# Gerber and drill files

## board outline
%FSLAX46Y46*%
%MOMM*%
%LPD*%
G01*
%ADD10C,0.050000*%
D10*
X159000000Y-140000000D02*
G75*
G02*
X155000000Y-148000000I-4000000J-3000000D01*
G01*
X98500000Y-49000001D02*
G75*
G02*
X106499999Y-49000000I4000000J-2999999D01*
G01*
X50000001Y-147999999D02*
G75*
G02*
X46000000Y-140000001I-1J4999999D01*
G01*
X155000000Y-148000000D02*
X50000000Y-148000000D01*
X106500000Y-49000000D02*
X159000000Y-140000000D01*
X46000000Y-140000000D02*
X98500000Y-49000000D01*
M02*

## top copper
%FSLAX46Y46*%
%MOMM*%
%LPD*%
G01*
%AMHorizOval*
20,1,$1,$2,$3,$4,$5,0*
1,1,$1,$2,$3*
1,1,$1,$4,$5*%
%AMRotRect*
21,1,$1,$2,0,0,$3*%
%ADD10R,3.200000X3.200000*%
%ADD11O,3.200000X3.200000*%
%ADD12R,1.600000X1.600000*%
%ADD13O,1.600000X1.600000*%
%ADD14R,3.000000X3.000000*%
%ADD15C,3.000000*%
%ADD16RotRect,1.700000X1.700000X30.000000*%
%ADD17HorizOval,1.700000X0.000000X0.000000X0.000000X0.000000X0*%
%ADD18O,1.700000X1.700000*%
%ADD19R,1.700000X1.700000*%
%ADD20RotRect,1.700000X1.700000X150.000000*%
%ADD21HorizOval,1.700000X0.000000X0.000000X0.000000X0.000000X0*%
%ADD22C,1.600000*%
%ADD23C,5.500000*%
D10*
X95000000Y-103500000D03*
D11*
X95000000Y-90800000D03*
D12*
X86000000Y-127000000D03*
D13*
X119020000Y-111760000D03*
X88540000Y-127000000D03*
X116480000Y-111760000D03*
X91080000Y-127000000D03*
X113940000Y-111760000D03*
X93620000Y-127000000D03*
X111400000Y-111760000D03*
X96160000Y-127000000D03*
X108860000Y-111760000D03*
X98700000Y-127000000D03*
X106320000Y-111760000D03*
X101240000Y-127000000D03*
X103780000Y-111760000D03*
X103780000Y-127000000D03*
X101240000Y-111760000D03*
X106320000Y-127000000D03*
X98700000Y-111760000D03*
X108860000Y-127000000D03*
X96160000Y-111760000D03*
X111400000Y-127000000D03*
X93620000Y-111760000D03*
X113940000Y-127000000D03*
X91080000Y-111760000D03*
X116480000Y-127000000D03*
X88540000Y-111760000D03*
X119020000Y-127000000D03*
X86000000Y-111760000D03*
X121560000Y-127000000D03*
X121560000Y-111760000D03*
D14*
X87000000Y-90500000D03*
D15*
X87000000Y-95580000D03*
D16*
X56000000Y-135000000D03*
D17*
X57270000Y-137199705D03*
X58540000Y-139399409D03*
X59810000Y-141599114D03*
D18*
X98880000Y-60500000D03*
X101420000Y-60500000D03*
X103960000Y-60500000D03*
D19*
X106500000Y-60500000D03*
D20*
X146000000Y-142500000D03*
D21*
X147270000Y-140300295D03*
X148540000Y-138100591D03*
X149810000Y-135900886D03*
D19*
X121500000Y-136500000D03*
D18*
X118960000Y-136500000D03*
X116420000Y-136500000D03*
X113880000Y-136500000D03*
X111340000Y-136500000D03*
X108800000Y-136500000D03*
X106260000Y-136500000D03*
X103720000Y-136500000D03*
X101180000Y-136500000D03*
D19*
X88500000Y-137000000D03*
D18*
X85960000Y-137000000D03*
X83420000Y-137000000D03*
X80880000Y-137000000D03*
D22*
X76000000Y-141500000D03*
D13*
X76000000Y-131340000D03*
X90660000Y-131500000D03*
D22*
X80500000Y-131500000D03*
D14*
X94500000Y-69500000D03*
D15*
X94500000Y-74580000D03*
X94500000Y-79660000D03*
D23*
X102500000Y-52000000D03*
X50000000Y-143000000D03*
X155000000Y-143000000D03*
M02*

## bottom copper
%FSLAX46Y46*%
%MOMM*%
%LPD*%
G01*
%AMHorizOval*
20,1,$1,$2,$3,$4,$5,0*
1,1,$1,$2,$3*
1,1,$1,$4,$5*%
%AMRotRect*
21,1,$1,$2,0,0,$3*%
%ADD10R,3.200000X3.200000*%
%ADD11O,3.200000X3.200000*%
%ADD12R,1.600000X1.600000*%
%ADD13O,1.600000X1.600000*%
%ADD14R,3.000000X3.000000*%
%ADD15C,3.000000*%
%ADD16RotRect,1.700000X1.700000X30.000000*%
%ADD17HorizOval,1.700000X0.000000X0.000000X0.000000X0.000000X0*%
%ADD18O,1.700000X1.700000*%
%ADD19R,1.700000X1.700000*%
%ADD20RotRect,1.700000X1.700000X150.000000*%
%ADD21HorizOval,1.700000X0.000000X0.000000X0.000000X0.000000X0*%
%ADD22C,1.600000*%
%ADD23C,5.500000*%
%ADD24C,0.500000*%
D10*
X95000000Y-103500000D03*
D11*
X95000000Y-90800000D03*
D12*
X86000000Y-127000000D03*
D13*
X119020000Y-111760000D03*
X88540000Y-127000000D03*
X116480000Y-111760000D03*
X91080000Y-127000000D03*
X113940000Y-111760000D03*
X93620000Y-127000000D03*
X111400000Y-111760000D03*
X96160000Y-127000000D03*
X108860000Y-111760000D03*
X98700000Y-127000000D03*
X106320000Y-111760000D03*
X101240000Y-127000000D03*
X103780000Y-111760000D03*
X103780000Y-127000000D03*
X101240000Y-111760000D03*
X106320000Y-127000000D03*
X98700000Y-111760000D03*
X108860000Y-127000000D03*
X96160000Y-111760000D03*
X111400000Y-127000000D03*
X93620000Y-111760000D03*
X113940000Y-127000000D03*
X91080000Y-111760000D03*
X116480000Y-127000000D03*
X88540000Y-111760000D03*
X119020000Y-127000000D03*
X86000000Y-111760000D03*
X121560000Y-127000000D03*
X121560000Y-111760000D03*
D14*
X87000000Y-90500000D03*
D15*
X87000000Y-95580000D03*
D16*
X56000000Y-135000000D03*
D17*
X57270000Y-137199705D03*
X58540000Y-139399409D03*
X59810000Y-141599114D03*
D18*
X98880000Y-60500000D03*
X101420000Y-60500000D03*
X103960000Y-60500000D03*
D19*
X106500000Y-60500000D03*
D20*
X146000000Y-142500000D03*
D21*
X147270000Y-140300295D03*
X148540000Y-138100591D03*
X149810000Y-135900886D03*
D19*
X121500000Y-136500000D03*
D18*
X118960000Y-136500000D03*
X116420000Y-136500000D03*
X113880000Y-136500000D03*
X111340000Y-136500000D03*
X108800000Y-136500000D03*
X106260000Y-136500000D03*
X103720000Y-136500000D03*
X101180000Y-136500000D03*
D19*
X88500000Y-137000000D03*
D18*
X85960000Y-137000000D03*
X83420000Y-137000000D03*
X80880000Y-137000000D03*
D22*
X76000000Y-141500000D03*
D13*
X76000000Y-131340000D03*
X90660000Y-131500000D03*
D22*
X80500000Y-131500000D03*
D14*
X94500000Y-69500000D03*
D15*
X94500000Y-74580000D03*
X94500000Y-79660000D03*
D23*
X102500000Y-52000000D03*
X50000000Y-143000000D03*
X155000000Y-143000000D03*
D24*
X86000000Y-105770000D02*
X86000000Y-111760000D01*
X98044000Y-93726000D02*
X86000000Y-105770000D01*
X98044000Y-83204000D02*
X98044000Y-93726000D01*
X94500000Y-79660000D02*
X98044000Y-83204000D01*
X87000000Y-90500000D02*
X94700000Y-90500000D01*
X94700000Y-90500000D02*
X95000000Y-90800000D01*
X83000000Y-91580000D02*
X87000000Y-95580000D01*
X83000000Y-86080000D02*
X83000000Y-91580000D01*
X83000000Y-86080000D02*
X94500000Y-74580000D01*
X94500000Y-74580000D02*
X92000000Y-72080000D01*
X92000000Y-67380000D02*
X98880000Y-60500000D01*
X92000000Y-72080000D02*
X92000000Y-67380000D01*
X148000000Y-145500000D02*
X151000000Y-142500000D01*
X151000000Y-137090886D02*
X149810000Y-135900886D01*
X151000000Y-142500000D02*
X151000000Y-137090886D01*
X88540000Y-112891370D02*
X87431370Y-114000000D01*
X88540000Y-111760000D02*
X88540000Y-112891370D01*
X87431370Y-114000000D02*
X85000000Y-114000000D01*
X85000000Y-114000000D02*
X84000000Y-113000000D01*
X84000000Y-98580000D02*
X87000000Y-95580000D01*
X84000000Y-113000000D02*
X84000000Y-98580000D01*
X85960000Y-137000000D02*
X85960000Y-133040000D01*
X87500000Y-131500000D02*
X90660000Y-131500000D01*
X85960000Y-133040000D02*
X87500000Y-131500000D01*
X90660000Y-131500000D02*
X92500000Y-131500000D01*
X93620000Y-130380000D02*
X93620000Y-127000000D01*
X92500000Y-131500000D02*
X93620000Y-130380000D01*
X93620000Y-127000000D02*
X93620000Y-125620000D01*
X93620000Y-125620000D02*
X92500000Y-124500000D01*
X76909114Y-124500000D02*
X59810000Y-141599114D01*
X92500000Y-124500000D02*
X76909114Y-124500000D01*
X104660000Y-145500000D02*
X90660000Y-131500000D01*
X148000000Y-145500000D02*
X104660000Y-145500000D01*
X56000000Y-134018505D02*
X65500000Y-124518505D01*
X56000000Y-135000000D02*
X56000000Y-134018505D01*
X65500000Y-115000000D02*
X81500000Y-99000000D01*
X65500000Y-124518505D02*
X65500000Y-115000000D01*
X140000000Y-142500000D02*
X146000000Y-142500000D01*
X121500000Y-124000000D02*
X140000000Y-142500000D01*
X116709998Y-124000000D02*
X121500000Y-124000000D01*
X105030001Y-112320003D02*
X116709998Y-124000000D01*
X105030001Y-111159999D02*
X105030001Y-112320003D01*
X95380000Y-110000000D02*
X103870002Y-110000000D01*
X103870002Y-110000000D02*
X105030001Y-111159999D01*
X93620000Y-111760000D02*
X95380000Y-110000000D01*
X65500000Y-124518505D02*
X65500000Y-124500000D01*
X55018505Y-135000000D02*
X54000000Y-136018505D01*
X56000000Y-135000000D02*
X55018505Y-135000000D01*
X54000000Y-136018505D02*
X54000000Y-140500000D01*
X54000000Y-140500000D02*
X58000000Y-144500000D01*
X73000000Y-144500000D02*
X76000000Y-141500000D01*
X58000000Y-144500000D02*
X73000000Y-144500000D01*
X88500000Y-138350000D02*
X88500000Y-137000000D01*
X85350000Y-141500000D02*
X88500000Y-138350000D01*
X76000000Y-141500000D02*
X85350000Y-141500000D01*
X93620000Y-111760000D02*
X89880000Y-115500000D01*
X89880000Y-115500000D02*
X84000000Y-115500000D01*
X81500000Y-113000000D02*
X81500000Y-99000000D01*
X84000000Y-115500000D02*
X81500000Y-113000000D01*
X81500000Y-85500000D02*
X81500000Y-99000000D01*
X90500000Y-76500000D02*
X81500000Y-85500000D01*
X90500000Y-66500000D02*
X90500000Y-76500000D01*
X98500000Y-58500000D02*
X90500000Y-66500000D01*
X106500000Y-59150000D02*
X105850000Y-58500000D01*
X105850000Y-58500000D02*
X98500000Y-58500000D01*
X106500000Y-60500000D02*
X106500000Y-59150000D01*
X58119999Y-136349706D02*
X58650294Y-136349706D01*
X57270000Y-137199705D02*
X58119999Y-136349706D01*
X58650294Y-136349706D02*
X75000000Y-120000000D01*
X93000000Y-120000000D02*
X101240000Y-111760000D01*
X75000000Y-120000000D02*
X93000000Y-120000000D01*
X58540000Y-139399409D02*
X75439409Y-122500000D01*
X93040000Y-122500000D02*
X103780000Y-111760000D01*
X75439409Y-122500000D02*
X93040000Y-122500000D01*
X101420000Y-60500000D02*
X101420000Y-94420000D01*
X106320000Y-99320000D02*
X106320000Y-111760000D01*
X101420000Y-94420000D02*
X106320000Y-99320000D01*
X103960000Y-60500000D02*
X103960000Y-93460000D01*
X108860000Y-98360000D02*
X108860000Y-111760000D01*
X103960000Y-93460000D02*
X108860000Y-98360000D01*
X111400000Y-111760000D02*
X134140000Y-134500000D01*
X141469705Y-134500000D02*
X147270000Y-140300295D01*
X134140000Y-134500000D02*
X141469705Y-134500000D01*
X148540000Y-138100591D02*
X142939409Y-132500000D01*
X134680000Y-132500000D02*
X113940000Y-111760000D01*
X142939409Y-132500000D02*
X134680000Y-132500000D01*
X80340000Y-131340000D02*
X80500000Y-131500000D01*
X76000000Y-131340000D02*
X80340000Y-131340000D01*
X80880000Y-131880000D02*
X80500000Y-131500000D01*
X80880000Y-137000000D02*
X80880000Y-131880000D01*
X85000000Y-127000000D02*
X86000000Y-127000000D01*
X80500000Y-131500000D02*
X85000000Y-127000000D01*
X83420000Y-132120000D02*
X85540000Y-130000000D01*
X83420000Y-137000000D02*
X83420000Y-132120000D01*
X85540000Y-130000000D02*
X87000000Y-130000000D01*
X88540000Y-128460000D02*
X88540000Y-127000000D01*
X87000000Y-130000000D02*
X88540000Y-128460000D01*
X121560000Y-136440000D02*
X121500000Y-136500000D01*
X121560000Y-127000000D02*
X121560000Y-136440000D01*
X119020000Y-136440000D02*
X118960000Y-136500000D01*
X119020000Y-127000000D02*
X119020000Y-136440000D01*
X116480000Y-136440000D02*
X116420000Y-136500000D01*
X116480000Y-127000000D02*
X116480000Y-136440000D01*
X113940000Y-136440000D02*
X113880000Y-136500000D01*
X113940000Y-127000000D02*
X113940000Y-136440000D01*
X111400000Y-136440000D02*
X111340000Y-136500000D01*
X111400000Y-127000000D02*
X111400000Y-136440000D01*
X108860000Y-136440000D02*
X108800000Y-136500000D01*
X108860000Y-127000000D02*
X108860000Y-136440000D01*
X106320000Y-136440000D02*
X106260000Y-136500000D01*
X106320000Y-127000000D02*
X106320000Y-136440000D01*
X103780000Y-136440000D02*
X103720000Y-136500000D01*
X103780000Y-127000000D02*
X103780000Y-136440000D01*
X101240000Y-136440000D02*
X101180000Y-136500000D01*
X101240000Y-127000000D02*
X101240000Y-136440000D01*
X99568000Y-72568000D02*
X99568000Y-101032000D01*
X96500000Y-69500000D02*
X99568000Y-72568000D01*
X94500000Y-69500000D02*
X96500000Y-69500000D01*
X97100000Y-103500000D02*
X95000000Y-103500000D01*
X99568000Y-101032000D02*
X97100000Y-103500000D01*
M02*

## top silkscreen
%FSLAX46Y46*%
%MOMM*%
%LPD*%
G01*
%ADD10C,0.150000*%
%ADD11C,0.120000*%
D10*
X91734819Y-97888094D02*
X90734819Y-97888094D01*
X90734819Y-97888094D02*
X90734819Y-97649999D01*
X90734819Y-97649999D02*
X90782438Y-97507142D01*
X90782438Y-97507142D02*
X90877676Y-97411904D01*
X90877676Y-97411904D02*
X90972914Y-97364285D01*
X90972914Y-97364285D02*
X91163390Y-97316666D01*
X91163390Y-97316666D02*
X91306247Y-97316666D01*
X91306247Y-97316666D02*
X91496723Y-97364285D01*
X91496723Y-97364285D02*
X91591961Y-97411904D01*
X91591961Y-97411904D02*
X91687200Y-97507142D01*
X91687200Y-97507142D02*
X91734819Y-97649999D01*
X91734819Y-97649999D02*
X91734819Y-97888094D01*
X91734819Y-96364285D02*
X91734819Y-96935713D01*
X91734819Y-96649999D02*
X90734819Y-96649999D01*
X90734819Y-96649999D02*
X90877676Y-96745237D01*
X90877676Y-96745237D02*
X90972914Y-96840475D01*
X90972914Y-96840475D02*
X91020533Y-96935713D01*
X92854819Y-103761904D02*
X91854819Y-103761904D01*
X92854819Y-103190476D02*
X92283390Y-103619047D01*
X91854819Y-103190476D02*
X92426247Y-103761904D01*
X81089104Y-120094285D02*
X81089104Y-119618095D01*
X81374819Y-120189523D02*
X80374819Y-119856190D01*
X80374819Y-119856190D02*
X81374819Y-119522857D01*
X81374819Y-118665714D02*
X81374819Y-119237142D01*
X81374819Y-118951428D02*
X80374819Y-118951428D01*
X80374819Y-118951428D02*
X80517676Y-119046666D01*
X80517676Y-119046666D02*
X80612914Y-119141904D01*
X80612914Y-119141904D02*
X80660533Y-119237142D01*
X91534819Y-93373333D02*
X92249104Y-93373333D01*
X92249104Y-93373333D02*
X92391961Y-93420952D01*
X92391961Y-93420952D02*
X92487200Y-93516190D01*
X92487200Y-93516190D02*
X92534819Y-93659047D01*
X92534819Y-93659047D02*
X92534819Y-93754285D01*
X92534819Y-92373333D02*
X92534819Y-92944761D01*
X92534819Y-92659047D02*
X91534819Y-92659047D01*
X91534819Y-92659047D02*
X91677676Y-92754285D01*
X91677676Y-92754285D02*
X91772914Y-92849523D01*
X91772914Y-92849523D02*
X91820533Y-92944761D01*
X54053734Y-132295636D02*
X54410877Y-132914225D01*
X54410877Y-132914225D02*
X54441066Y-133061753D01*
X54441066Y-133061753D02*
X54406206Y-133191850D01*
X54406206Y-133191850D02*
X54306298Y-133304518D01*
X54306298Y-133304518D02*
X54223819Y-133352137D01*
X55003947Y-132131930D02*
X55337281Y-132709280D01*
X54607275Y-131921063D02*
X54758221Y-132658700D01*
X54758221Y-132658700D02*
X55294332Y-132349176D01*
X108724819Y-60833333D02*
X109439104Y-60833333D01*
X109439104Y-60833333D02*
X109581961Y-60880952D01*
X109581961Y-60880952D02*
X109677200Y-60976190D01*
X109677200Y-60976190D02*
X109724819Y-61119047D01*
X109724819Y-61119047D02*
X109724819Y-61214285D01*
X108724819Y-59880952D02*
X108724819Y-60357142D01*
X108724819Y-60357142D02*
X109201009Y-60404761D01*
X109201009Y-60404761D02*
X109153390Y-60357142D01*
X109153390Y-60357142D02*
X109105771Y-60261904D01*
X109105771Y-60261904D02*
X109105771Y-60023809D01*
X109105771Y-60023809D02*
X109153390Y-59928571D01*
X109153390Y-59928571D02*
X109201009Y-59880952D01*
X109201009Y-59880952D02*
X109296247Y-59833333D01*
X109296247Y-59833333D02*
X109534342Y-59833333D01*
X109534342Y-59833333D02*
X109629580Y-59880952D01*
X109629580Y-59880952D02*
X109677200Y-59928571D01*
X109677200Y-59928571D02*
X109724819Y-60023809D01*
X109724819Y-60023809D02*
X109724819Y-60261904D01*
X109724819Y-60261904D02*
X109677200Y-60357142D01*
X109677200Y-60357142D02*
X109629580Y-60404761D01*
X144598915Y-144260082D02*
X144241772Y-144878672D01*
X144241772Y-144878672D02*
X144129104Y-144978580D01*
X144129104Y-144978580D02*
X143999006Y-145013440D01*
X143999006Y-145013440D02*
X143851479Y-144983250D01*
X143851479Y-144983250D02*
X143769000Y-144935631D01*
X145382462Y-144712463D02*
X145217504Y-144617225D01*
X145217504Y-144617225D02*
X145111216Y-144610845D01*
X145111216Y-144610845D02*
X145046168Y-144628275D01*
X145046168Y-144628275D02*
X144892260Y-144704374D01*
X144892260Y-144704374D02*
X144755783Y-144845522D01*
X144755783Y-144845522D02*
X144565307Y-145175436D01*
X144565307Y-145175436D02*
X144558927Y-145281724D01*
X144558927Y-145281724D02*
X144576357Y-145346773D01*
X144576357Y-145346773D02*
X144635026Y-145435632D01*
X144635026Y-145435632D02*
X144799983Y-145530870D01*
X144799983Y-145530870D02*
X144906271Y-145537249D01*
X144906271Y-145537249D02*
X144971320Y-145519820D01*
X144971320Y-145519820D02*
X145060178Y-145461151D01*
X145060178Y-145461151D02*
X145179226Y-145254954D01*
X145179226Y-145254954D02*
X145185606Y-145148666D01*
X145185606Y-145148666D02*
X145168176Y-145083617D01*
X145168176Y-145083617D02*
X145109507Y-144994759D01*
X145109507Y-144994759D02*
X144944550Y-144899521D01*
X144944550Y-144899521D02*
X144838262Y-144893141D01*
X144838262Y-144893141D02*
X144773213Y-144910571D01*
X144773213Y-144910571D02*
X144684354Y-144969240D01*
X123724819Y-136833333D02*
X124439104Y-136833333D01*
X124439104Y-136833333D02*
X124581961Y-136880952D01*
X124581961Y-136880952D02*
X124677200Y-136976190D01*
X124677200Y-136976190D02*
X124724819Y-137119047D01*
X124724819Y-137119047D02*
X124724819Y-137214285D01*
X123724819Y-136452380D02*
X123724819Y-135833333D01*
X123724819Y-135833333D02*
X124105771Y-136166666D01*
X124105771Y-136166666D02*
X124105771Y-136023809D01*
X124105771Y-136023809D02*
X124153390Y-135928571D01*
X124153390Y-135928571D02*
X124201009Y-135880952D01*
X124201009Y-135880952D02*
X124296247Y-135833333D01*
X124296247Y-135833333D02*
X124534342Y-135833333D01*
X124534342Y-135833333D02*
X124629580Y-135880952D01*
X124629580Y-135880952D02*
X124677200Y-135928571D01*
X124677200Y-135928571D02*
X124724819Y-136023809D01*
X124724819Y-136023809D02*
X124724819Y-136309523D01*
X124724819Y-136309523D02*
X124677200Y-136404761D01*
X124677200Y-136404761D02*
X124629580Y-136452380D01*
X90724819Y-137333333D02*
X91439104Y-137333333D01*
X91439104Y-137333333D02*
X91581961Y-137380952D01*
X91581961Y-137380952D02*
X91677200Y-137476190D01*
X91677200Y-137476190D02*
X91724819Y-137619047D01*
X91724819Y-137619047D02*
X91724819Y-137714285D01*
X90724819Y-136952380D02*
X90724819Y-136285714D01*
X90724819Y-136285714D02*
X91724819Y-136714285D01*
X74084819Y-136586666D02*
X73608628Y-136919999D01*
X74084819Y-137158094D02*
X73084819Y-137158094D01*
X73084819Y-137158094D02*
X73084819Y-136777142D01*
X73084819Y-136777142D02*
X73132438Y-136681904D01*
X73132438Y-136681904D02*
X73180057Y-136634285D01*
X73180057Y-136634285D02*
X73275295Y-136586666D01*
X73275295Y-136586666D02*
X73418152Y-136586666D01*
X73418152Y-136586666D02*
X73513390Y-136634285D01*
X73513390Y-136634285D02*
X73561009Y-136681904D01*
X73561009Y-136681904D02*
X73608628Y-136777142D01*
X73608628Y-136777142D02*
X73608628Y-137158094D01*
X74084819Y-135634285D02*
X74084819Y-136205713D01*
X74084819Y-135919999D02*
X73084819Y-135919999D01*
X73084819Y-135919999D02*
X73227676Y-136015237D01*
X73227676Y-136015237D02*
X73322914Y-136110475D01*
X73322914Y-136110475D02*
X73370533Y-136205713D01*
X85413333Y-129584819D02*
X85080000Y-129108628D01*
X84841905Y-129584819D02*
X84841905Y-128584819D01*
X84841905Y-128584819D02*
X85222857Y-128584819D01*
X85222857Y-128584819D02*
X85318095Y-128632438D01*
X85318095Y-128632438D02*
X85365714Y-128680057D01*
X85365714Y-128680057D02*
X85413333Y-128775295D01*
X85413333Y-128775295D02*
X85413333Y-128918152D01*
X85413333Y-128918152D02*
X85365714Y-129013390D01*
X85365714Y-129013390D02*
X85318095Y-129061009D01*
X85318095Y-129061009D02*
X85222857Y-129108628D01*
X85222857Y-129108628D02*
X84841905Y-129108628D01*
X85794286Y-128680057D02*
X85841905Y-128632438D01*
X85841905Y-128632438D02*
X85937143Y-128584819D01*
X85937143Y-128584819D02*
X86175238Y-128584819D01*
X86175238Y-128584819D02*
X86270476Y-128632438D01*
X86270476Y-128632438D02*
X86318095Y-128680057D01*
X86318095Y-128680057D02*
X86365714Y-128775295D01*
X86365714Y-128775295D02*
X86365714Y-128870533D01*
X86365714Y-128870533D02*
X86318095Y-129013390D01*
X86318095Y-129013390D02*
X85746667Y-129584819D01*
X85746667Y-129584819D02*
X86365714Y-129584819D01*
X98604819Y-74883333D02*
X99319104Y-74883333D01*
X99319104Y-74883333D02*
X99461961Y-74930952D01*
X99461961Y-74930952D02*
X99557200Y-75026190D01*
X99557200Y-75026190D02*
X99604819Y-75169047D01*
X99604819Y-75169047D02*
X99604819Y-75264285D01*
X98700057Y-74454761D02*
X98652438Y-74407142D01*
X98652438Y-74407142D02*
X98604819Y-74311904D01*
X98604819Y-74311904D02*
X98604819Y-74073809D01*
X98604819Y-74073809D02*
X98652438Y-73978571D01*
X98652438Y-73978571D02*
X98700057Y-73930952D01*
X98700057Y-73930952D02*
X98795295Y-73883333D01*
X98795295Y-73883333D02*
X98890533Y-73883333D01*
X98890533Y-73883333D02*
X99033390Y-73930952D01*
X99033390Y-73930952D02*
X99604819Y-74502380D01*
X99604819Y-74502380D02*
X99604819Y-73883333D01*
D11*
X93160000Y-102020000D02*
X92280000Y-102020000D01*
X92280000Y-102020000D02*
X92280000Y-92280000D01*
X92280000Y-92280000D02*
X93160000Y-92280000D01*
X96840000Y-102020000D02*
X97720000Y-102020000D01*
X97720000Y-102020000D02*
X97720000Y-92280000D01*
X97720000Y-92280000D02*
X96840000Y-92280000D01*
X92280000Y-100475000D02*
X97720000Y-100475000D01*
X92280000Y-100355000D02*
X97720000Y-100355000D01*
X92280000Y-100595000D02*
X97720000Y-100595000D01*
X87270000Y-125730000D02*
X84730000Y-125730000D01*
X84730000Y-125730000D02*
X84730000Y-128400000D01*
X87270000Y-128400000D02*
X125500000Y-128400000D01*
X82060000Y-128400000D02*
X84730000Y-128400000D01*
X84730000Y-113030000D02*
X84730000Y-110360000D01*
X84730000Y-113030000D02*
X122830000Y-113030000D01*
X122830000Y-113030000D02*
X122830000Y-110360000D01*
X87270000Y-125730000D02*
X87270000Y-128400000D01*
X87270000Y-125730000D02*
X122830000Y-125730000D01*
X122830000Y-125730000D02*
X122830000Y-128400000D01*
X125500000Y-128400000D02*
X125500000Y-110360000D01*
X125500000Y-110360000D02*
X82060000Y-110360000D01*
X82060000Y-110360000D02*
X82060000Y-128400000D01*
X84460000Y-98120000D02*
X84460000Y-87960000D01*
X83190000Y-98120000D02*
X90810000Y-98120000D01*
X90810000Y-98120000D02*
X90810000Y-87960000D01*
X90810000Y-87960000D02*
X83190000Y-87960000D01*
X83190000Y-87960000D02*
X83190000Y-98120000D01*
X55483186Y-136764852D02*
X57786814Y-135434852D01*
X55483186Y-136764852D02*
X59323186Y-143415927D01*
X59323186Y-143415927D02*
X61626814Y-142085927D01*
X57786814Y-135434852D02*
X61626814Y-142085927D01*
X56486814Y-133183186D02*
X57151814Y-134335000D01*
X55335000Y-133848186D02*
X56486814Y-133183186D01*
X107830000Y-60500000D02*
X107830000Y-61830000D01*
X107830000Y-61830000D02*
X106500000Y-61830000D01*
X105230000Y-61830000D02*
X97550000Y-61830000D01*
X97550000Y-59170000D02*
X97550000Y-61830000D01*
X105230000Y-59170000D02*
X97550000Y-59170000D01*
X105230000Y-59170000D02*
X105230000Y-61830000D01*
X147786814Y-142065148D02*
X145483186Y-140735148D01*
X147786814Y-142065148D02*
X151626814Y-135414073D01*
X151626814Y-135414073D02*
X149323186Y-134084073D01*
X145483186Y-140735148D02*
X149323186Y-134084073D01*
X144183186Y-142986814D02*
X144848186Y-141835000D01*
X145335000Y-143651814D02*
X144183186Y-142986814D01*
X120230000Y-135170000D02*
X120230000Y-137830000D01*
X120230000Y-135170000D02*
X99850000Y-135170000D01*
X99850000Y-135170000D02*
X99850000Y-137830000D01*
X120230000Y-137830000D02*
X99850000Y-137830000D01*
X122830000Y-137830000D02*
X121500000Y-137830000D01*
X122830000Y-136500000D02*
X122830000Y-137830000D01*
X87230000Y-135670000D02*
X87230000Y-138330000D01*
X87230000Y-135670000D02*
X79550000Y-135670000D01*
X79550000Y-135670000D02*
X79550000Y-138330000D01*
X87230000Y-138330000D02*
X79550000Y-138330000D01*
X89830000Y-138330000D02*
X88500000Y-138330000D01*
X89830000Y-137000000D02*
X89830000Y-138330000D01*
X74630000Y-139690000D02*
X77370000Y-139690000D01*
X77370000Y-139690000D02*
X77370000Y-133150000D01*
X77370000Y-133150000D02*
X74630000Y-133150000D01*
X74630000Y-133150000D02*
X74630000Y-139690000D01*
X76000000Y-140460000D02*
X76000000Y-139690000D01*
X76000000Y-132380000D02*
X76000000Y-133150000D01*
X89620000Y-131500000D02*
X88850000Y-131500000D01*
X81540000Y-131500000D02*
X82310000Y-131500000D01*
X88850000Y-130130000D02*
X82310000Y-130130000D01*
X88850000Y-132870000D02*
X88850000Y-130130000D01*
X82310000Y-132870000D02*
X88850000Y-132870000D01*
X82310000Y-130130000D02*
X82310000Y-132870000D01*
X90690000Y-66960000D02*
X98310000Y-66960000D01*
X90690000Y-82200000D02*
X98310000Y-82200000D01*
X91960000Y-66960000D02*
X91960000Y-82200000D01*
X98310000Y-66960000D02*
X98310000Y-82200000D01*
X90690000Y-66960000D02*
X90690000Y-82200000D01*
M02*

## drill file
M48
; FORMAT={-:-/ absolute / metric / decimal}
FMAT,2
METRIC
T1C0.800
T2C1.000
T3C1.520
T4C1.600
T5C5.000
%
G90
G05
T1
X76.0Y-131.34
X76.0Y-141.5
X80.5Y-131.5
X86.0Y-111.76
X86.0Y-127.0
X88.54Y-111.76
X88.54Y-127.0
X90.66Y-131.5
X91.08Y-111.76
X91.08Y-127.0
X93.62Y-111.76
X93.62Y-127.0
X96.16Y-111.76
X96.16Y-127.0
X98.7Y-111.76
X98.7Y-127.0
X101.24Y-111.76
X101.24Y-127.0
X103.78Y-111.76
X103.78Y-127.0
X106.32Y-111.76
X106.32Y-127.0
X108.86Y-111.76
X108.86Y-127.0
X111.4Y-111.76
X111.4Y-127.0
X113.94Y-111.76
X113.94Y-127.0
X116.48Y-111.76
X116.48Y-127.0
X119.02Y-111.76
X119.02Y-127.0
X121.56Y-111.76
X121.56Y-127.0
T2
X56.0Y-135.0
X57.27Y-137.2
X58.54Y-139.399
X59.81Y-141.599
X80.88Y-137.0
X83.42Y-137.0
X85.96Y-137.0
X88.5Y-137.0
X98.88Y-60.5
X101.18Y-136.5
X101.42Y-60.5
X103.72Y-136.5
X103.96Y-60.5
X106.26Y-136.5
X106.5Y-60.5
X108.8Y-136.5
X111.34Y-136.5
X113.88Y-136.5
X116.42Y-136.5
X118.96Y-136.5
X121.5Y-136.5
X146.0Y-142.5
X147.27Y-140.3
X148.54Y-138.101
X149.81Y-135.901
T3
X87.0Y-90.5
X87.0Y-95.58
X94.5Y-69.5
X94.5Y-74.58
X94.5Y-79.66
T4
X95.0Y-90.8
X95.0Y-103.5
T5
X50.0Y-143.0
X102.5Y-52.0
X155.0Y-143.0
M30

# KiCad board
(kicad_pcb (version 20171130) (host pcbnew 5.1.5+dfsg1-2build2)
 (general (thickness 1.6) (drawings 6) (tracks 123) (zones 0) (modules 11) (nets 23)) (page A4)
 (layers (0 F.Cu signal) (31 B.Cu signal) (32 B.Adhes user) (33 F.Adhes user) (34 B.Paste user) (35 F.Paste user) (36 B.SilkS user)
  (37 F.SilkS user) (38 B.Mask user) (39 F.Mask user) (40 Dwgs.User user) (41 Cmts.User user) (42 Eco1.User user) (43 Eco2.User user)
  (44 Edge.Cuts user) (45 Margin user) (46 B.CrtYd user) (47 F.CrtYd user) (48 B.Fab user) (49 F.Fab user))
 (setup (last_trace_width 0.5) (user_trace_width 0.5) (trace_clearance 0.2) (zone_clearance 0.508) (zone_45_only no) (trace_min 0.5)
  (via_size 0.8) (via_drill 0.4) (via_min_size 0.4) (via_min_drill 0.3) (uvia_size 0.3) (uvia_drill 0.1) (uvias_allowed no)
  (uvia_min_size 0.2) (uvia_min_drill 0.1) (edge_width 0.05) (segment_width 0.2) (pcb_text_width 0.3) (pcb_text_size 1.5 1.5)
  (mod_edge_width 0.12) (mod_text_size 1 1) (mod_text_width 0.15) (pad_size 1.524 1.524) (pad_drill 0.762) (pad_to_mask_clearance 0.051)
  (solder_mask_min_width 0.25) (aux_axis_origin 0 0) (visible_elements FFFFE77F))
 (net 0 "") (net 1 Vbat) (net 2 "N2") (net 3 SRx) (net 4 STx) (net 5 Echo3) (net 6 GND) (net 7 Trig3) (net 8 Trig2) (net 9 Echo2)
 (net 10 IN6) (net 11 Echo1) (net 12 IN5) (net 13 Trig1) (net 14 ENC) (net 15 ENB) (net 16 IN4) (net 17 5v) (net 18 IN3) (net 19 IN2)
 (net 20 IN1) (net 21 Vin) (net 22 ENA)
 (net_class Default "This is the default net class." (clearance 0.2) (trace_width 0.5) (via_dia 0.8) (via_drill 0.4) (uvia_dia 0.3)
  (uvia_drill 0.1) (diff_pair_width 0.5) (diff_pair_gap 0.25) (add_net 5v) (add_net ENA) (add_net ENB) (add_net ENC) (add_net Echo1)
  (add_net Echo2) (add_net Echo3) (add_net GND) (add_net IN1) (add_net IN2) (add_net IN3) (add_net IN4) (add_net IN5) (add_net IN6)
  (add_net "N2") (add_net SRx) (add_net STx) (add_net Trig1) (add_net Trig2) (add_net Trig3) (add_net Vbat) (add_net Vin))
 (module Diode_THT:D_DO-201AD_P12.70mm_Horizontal (layer F.Cu) (at 95 103.5 90)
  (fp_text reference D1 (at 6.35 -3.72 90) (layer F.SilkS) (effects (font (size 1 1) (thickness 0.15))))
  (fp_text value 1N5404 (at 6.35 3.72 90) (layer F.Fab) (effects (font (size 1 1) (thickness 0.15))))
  (fp_line (start 1.48 -1.84) (end 1.48 -2.72) (layer F.SilkS) (width 0.12))
  (fp_line (start 1.48 -2.72) (end 11.22 -2.72) (layer F.SilkS) (width 0.12))
  (fp_line (start 11.22 -2.72) (end 11.22 -1.84) (layer F.SilkS) (width 0.12))
  (fp_line (start 1.48 1.84) (end 1.48 2.72) (layer F.SilkS) (width 0.12))
  (fp_line (start 1.48 2.72) (end 11.22 2.72) (layer F.SilkS) (width 0.12))
  (fp_line (start 11.22 2.72) (end 11.22 1.84) (layer F.SilkS) (width 0.12))
  (fp_line (start 3.025 -2.72) (end 3.025 2.72) (layer F.SilkS) (width 0.12))
  (fp_line (start 3.145 -2.72) (end 3.145 2.72) (layer F.SilkS) (width 0.12))
  (fp_line (start 2.905 -2.72) (end 2.905 2.72) (layer F.SilkS) (width 0.12))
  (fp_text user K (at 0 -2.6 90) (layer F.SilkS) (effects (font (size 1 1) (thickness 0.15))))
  (pad 1 thru_hole rect (at 0 0 90) (size 3.2 3.2) (drill 1.6) (layers *.Cu *.Mask) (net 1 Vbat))
  (pad 2 thru_hole oval (at 12.7 0 90) (size 3.2 3.2) (drill 1.6) (layers *.Cu *.Mask) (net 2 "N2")))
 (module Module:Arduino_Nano (layer F.Cu) (at 86 127 90)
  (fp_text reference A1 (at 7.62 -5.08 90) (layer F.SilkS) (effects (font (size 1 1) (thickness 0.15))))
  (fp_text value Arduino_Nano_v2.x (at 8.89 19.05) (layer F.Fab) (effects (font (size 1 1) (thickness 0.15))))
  (fp_line (start 1.27 1.27) (end 1.27 -1.27) (layer F.SilkS) (width 0.12))
  (fp_line (start 1.27 -1.27) (end -1.4 -1.27) (layer F.SilkS) (width 0.12))
  (fp_line (start -1.4 1.27) (end -1.4 39.5) (layer F.SilkS) (width 0.12))
  (fp_line (start -1.4 -3.94) (end -1.4 -1.27) (layer F.SilkS) (width 0.12))
  (fp_line (start 13.97 -1.27) (end 16.64 -1.27) (layer F.SilkS) (width 0.12))
  (fp_line (start 13.97 -1.27) (end 13.97 36.83) (layer F.SilkS) (width 0.12))
  (fp_line (start 13.97 36.83) (end 16.64 36.83) (layer F.SilkS) (width 0.12))
  (fp_line (start 1.27 1.27) (end -1.4 1.27) (layer F.SilkS) (width 0.12))
  (fp_line (start 1.27 1.27) (end 1.27 36.83) (layer F.SilkS) (width 0.12))
  (fp_line (start 1.27 36.83) (end -1.4 36.83) (layer F.SilkS) (width 0.12))
  (fp_line (start -1.4 39.5) (end 16.64 39.5) (layer F.SilkS) (width 0.12))
  (fp_line (start 16.64 39.5) (end 16.64 -3.94) (layer F.SilkS) (width 0.12))
  (fp_line (start 16.64 -3.94) (end -1.4 -3.94) (layer F.SilkS) (width 0.12))
  (pad 1 thru_hole rect (at 0 0 90) (size 1.6 1.6) (drill 0.8) (layers *.Cu *.Mask) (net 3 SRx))
  (pad 17 thru_hole oval (at 15.24 33.02 90) (size 1.6 1.6) (drill 0.8) (layers *.Cu *.Mask))
  (pad 2 thru_hole oval (at 0 2.54 90) (size 1.6 1.6) (drill 0.8) (layers *.Cu *.Mask) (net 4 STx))
  (pad 18 thru_hole oval (at 15.24 30.48 90) (size 1.6 1.6) (drill 0.8) (layers *.Cu *.Mask))
  (pad 3 thru_hole oval (at 0 5.08 90) (size 1.6 1.6) (drill 0.8) (layers *.Cu *.Mask))
  (pad 19 thru_hole oval (at 15.24 27.94 90) (size 1.6 1.6) (drill 0.8) (layers *.Cu *.Mask) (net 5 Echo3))
  (pad 4 thru_hole oval (at 0 7.62 90) (size 1.6 1.6) (drill 0.8) (layers *.Cu *.Mask) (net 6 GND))
  (pad 20 thru_hole oval (at 15.24 25.4 90) (size 1.6 1.6) (drill 0.8) (layers *.Cu *.Mask) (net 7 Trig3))
  (pad 5 thru_hole oval (at 0 10.16 90) (size 1.6 1.6) (drill 0.8) (layers *.Cu *.Mask))
  (pad 21 thru_hole oval (at 15.24 22.86 90) (size 1.6 1.6) (drill 0.8) (layers *.Cu *.Mask) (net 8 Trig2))
  (pad 6 thru_hole oval (at 0 12.7 90) (size 1.6 1.6) (drill 0.8) (layers *.Cu *.Mask))
  (pad 22 thru_hole oval (at 15.24 20.32 90) (size 1.6 1.6) (drill 0.8) (layers *.Cu *.Mask) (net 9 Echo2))
  (pad 7 thru_hole oval (at 0 15.24 90) (size 1.6 1.6) (drill 0.8) (layers *.Cu *.Mask) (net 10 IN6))
  (pad 23 thru_hole oval (at 15.24 17.78 90) (size 1.6 1.6) (drill 0.8) (layers *.Cu *.Mask) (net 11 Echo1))
  (pad 8 thru_hole oval (at 0 17.78 90) (size 1.6 1.6) (drill 0.8) (layers *.Cu *.Mask) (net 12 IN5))
  (pad 24 thru_hole oval (at 15.24 15.24 90) (size 1.6 1.6) (drill 0.8) (layers *.Cu *.Mask) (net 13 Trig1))
  (pad 9 thru_hole oval (at 0 20.32 90) (size 1.6 1.6) (drill 0.8) (layers *.Cu *.Mask) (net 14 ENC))
  (pad 25 thru_hole oval (at 15.24 12.7 90) (size 1.6 1.6) (drill 0.8) (layers *.Cu *.Mask))
  (pad 10 thru_hole oval (at 0 22.86 90) (size 1.6 1.6) (drill 0.8) (layers *.Cu *.Mask) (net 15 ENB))
  (pad 26 thru_hole oval (at 15.24 10.16 90) (size 1.6 1.6) (drill 0.8) (layers *.Cu *.Mask))
  (pad 11 thru_hole oval (at 0 25.4 90) (size 1.6 1.6) (drill 0.8) (layers *.Cu *.Mask) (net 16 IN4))
  (pad 27 thru_hole oval (at 15.24 7.62 90) (size 1.6 1.6) (drill 0.8) (layers *.Cu *.Mask) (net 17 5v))
  (pad 12 thru_hole oval (at 0 27.94 90) (size 1.6 1.6) (drill 0.8) (layers *.Cu *.Mask) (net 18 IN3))
  (pad 28 thru_hole oval (at 15.24 5.08 90) (size 1.6 1.6) (drill 0.8) (layers *.Cu *.Mask))
  (pad 13 thru_hole oval (at 0 30.48 90) (size 1.6 1.6) (drill 0.8) (layers *.Cu *.Mask) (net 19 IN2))
  (pad 29 thru_hole oval (at 15.24 2.54 90) (size 1.6 1.6) (drill 0.8) (layers *.Cu *.Mask) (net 6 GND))
  (pad 14 thru_hole oval (at 0 33.02 90) (size 1.6 1.6) (drill 0.8) (layers *.Cu *.Mask) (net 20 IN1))
  (pad 30 thru_hole oval (at 15.24 0 90) (size 1.6 1.6) (drill 0.8) (layers *.Cu *.Mask) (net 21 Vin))
  (pad 15 thru_hole oval (at 0 35.56 90) (size 1.6 1.6) (drill 0.8) (layers *.Cu *.Mask) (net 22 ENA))
  (pad 16 thru_hole oval (at 15.24 35.56 90) (size 1.6 1.6) (drill 0.8) (layers *.Cu *.Mask)))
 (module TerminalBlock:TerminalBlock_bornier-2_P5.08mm (layer F.Cu) (at 87 90.5 270)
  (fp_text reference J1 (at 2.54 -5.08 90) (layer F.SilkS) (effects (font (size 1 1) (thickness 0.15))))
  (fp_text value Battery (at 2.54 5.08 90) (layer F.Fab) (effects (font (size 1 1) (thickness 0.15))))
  (fp_line (start 7.62 2.54) (end -2.54 2.54) (layer F.SilkS) (width 0.12))
  (fp_line (start 7.62 3.81) (end 7.62 -3.81) (layer F.SilkS) (width 0.12))
  (fp_line (start 7.62 -3.81) (end -2.54 -3.81) (layer F.SilkS) (width 0.12))
  (fp_line (start -2.54 -3.81) (end -2.54 3.81) (layer F.SilkS) (width 0.12))
  (fp_line (start -2.54 3.81) (end 7.62 3.81) (layer F.SilkS) (width 0.12))
  (pad 1 thru_hole rect (at 0 0 270) (size 3 3) (drill 1.52) (layers *.Cu *.Mask) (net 2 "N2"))
  (pad 2 thru_hole circle (at 5.08 0 270) (size 3 3) (drill 1.52) (layers *.Cu *.Mask) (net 6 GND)))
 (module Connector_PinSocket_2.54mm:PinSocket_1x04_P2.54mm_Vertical (layer F.Cu) (at 56 135 30)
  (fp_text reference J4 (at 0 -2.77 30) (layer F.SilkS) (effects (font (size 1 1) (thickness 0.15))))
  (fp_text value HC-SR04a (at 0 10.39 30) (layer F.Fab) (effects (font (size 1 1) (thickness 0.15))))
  (fp_line (start -1.33 1.27) (end 1.33 1.27) (layer F.SilkS) (width 0.12))
  (fp_line (start -1.33 1.27) (end -1.33 8.95) (layer F.SilkS) (width 0.12))
  (fp_line (start -1.33 8.95) (end 1.33 8.95) (layer F.SilkS) (width 0.12))
  (fp_line (start 1.33 1.27) (end 1.33 8.95) (layer F.SilkS) (width 0.12))
  (fp_line (start 1.33 -1.33) (end 1.33 0) (layer F.SilkS) (width 0.12))
  (fp_line (start 0 -1.33) (end 1.33 -1.33) (layer F.SilkS) (width 0.12))
  (pad 1 thru_hole rect (at 0 0 30) (size 1.7 1.7) (drill 1) (layers *.Cu *.Mask) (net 17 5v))
  (pad 2 thru_hole oval (at 0 2.54 30) (size 1.7 1.7) (drill 1) (layers *.Cu *.Mask) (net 13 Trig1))
  (pad 3 thru_hole oval (at 0 5.08 30) (size 1.7 1.7) (drill 1) (layers *.Cu *.Mask) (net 11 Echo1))
  (pad 4 thru_hole oval (at 0 7.62 30) (size 1.7 1.7) (drill 1) (layers *.Cu *.Mask) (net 6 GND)))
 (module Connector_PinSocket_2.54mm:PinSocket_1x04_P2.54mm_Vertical (layer F.Cu) (at 106.5 60.5 270)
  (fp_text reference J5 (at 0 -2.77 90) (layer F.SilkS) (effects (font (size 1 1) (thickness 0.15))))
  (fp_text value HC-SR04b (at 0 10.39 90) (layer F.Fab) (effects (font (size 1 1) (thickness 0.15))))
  (fp_line (start 0 -1.33) (end 1.33 -1.33) (layer F.SilkS) (width 0.12))
  (fp_line (start 1.33 -1.33) (end 1.33 0) (layer F.SilkS) (width 0.12))
  (fp_line (start 1.33 1.27) (end 1.33 8.95) (layer F.SilkS) (width 0.12))
  (fp_line (start -1.33 8.95) (end 1.33 8.95) (layer F.SilkS) (width 0.12))
  (fp_line (start -1.33 1.27) (end -1.33 8.95) (layer F.SilkS) (width 0.12))
  (fp_line (start -1.33 1.27) (end 1.33 1.27) (layer F.SilkS) (width 0.12))
  (pad 4 thru_hole oval (at 0 7.62 270) (size 1.7 1.7) (drill 1) (layers *.Cu *.Mask) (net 6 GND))
  (pad 3 thru_hole oval (at 0 5.08 270) (size 1.7 1.7) (drill 1) (layers *.Cu *.Mask) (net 9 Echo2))
  (pad 2 thru_hole oval (at 0 2.54 270) (size 1.7 1.7) (drill 1) (layers *.Cu *.Mask) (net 8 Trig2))
  (pad 1 thru_hole rect (at 0 0 270) (size 1.7 1.7) (drill 1) (layers *.Cu *.Mask) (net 17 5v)))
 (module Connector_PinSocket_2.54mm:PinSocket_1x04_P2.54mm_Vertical (layer F.Cu) (at 146 142.5 150)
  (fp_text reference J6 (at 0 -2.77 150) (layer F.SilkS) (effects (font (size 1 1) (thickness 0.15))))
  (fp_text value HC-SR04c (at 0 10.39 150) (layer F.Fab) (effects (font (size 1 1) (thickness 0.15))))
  (fp_line (start -1.33 1.27) (end 1.33 1.27) (layer F.SilkS) (width 0.12))
  (fp_line (start -1.33 1.27) (end -1.33 8.95) (layer F.SilkS) (width 0.12))
  (fp_line (start -1.33 8.95) (end 1.33 8.95) (layer F.SilkS) (width 0.12))
  (fp_line (start 1.33 1.27) (end 1.33 8.95) (layer F.SilkS) (width 0.12))
  (fp_line (start 1.33 -1.33) (end 1.33 0) (layer F.SilkS) (width 0.12))
  (fp_line (start 0 -1.33) (end 1.33 -1.33) (layer F.SilkS) (width 0.12))
  (pad 1 thru_hole rect (at 0 0 150) (size 1.7 1.7) (drill 1) (layers *.Cu *.Mask) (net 17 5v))
  (pad 2 thru_hole oval (at 0 2.54 150) (size 1.7 1.7) (drill 1) (layers *.Cu *.Mask) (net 7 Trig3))
  (pad 3 thru_hole oval (at 0 5.08 150) (size 1.7 1.7) (drill 1) (layers *.Cu *.Mask) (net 5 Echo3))
  (pad 4 thru_hole oval (at 0 7.62 150) (size 1.7 1.7) (drill 1) (layers *.Cu *.Mask) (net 6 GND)))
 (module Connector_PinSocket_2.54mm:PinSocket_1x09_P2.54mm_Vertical (layer F.Cu) (at 121.5 136.5 270)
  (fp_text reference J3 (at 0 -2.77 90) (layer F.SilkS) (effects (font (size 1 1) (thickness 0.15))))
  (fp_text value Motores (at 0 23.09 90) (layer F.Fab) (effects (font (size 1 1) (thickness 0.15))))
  (fp_line (start -1.33 1.27) (end 1.33 1.27) (layer F.SilkS) (width 0.12))
  (fp_line (start -1.33 1.27) (end -1.33 21.65) (layer F.SilkS) (width 0.12))
  (fp_line (start -1.33 21.65) (end 1.33 21.65) (layer F.SilkS) (width 0.12))
  (fp_line (start 1.33 1.27) (end 1.33 21.65) (layer F.SilkS) (width 0.12))
  (fp_line (start 1.33 -1.33) (end 1.33 0) (layer F.SilkS) (width 0.12))
  (fp_line (start 0 -1.33) (end 1.33 -1.33) (layer F.SilkS) (width 0.12))
  (pad 1 thru_hole rect (at 0 0 270) (size 1.7 1.7) (drill 1) (layers *.Cu *.Mask) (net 22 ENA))
  (pad 2 thru_hole oval (at 0 2.54 270) (size 1.7 1.7) (drill 1) (layers *.Cu *.Mask) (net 20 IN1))
  (pad 3 thru_hole oval (at 0 5.08 270) (size 1.7 1.7) (drill 1) (layers *.Cu *.Mask) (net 19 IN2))
  (pad 4 thru_hole oval (at 0 7.62 270) (size 1.7 1.7) (drill 1) (layers *.Cu *.Mask) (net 18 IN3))
  (pad 5 thru_hole oval (at 0 10.16 270) (size 1.7 1.7) (drill 1) (layers *.Cu *.Mask) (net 16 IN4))
  (pad 6 thru_hole oval (at 0 12.7 270) (size 1.7 1.7) (drill 1) (layers *.Cu *.Mask) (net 15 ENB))
  (pad 7 thru_hole oval (at 0 15.24 270) (size 1.7 1.7) (drill 1) (layers *.Cu *.Mask) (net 14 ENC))
  (pad 8 thru_hole oval (at 0 17.78 270) (size 1.7 1.7) (drill 1) (layers *.Cu *.Mask) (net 12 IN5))
  (pad 9 thru_hole oval (at 0 20.32 270) (size 1.7 1.7) (drill 1) (layers *.Cu *.Mask) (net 10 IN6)))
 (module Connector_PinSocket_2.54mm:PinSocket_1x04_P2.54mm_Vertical (layer F.Cu) (at 88.5 137 270)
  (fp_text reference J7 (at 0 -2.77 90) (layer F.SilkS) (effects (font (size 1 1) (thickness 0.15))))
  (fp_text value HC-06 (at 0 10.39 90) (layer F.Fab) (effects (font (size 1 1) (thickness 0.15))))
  (fp_line (start -1.33 1.27) (end 1.33 1.27) (layer F.SilkS) (width 0.12))
  (fp_line (start -1.33 1.27) (end -1.33 8.95) (layer F.SilkS) (width 0.12))
  (fp_line (start -1.33 8.95) (end 1.33 8.95) (layer F.SilkS) (width 0.12))
  (fp_line (start 1.33 1.27) (end 1.33 8.95) (layer F.SilkS) (width 0.12))
  (fp_line (start 1.33 -1.33) (end 1.33 0) (layer F.SilkS) (width 0.12))
  (fp_line (start 0 -1.33) (end 1.33 -1.33) (layer F.SilkS) (width 0.12))
  (pad 1 thru_hole rect (at 0 0 270) (size 1.7 1.7) (drill 1) (layers *.Cu *.Mask) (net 17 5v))
  (pad 2 thru_hole oval (at 0 2.54 270) (size 1.7 1.7) (drill 1) (layers *.Cu *.Mask) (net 6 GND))
  (pad 3 thru_hole oval (at 0 5.08 270) (size 1.7 1.7) (drill 1) (layers *.Cu *.Mask) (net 4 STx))
  (pad 4 thru_hole oval (at 0 7.62 270) (size 1.7 1.7) (drill 1) (layers *.Cu *.Mask) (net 3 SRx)))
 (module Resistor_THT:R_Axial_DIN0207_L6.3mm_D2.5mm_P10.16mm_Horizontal (layer F.Cu) (at 76 141.5 90)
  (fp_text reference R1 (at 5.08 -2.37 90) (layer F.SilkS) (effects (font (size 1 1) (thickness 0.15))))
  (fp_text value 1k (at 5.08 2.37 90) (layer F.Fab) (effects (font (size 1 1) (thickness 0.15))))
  (fp_line (start 1.81 -1.37) (end 1.81 1.37) (layer F.SilkS) (width 0.12))
  (fp_line (start 1.81 1.37) (end 8.35 1.37) (layer F.SilkS) (width 0.12))
  (fp_line (start 8.35 1.37) (end 8.35 -1.37) (layer F.SilkS) (width 0.12))
  (fp_line (start 8.35 -1.37) (end 1.81 -1.37) (layer F.SilkS) (width 0.12))
  (fp_line (start 1.04 0) (end 1.81 0) (layer F.SilkS) (width 0.12))
  (fp_line (start 9.12 0) (end 8.35 0) (layer F.SilkS) (width 0.12))
  (pad 1 thru_hole circle (at 0 0 90) (size 1.6 1.6) (drill 0.8) (layers *.Cu *.Mask) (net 17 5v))
  (pad 2 thru_hole oval (at 10.16 0 90) (size 1.6 1.6) (drill 0.8) (layers *.Cu *.Mask) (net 3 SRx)))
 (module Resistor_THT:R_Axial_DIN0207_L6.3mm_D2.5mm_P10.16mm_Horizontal (layer F.Cu) (at 80.5 131.5)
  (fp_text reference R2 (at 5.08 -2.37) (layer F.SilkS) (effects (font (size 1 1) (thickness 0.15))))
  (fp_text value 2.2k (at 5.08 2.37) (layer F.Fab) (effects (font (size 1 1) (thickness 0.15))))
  (fp_line (start 9.12 0) (end 8.35 0) (layer F.SilkS) (width 0.12))
  (fp_line (start 1.04 0) (end 1.81 0) (layer F.SilkS) (width 0.12))
  (fp_line (start 8.35 -1.37) (end 1.81 -1.37) (layer F.SilkS) (width 0.12))
  (fp_line (start 8.35 1.37) (end 8.35 -1.37) (layer F.SilkS) (width 0.12))
  (fp_line (start 1.81 1.37) (end 8.35 1.37) (layer F.SilkS) (width 0.12))
  (fp_line (start 1.81 -1.37) (end 1.81 1.37) (layer F.SilkS) (width 0.12))
  (pad 2 thru_hole oval (at 10.16 0) (size 1.6 1.6) (drill 0.8) (layers *.Cu *.Mask) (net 6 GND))
  (pad 1 thru_hole circle (at 0 0) (size 1.6 1.6) (drill 0.8) (layers *.Cu *.Mask) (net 3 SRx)))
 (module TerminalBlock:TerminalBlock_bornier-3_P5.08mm (layer F.Cu) (at 94.5 69.5 270)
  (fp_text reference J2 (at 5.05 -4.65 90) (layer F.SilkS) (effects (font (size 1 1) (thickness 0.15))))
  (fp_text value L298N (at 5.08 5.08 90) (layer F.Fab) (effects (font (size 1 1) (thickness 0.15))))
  (fp_line (start -2.54 3.81) (end -2.54 -3.81) (layer F.SilkS) (width 0.12))
  (fp_line (start 12.7 3.81) (end 12.7 -3.81) (layer F.SilkS) (width 0.12))
  (fp_line (start -2.54 2.54) (end 12.7 2.54) (layer F.SilkS) (width 0.12))
  (fp_line (start -2.54 -3.81) (end 12.7 -3.81) (layer F.SilkS) (width 0.12))
  (fp_line (start -2.54 3.81) (end 12.7 3.81) (layer F.SilkS) (width 0.12))
  (pad 1 thru_hole rect (at 0 0 270) (size 3 3) (drill 1.52) (layers *.Cu *.Mask) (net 1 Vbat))
  (pad 2 thru_hole circle (at 5.08 0 270) (size 3 3) (drill 1.52) (layers *.Cu *.Mask) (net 6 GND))
  (pad 3 thru_hole circle (at 10.16 0 270) (size 3 3) (drill 1.52) (layers *.Cu *.Mask) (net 21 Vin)))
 (gr_arc (start 155 143) (end 155 148) (angle -126.8698976) (layer Edge.Cuts) (width 0.05))
 (gr_arc (start 102.5 52) (end 106.499999 49) (angle -106.2602047) (layer Edge.Cuts) (width 0.05))
 (gr_arc (start 50 143) (end 46 140.000001) (angle -126.8698976) (layer Edge.Cuts) (width 0.05))
 (gr_line (start 155 148) (end 50 148) (layer Edge.Cuts) (width 0.05))
 (gr_line (start 106.5 49) (end 159 140) (layer Edge.Cuts) (width 0.05))
 (gr_line (start 46 140) (end 98.5 49) (layer Edge.Cuts) (width 0.05))
 (via (at 102.5 52) (size 5.5) (drill 5) (layers F.Cu B.Cu) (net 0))
 (via (at 50 143) (size 5.5) (drill 5) (layers F.Cu B.Cu) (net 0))
 (via (at 155 143) (size 5.5) (drill 5) (layers F.Cu B.Cu) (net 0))
 (segment (start 86 105.77) (end 86 111.76) (width 0.5) (layer B.Cu) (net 21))
 (segment (start 98.044 93.726) (end 86 105.77) (width 0.5) (layer B.Cu) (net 21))
 (segment (start 98.044 83.204) (end 98.044 93.726) (width 0.5) (layer B.Cu) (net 21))
 (segment (start 94.5 79.66) (end 98.044 83.204) (width 0.5) (layer B.Cu) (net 21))
 (segment (start 87 90.5) (end 94.7 90.5) (width 0.5) (layer B.Cu) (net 2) (status 30))
 (segment (start 94.7 90.5) (end 95 90.8) (width 0.5) (layer B.Cu) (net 2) (status 30))
 (segment (start 83 91.58) (end 87 95.58) (width 0.5) (layer B.Cu) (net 6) (status 20))
 (segment (start 83 86.08) (end 83 91.58) (width 0.5) (layer B.Cu) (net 6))
 (segment (start 83 86.08) (end 94.5 74.58) (width 0.5) (layer B.Cu) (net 6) (status 20))
 (segment (start 94.5 74.58) (end 92 72.08) (width 0.5) (layer B.Cu) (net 6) (status 10))
 (segment (start 92 67.38) (end 98.88 60.5) (width 0.5) (layer B.Cu) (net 6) (status 20))
 (segment (start 92 72.08) (end 92 67.38) (width 0.5) (layer B.Cu) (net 6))
 (segment (start 148 145.5) (end 151 142.5) (width 0.5) (layer B.Cu) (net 6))
 (segment (start 151 137.090886) (end 149.81 135.900886) (width 0.5) (layer B.Cu) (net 6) (status 20))
 (segment (start 151 142.5) (end 151 137.090886) (width 0.5) (layer B.Cu) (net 6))
 (segment (start 88.54 112.89137) (end 87.43137 114) (width 0.5) (layer B.Cu) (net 6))
 (segment (start 88.54 111.76) (end 88.54 112.89137) (width 0.5) (layer B.Cu) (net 6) (status 10))
 (segment (start 87.43137 114) (end 85 114) (width 0.5) (layer B.Cu) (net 6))
 (segment (start 85 114) (end 84 113) (width 0.5) (layer B.Cu) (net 6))
 (segment (start 84 98.58) (end 87 95.58) (width 0.5) (layer B.Cu) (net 6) (status 20))
 (segment (start 84 113) (end 84 98.58) (width 0.5) (layer B.Cu) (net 6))
 (segment (start 85.96 137) (end 85.96 133.04) (width 0.5) (layer B.Cu) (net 6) (status 10))
 (segment (start 87.5 131.5) (end 90.66 131.5) (width 0.5) (layer B.Cu) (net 6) (status 20))
 (segment (start 85.96 133.04) (end 87.5 131.5) (width 0.5) (layer B.Cu) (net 6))
 (segment (start 90.66 131.5) (end 92.5 131.5) (width 0.5) (layer B.Cu) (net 6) (status 10))
 (segment (start 93.62 130.38) (end 93.62 127) (width 0.5) (layer B.Cu) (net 6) (status 20))
 (segment (start 92.5 131.5) (end 93.62 130.38) (width 0.5) (layer B.Cu) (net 6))
 (segment (start 93.62 127) (end 93.62 125.62) (width 0.5) (layer B.Cu) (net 6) (status 10))
 (segment (start 93.62 125.62) (end 92.5 124.5) (width 0.5) (layer B.Cu) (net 6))
 (segment (start 76.909114 124.5) (end 59.81 141.599114) (width 0.5) (layer B.Cu) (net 6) (status 20))
 (segment (start 92.5 124.5) (end 76.909114 124.5) (width 0.5) (layer B.Cu) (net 6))
 (segment (start 104.66 145.5) (end 90.66 131.5) (width 0.5) (layer B.Cu) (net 6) (status 20))
 (segment (start 148 145.5) (end 104.66 145.5) (width 0.5) (layer B.Cu) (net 6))
 (segment (start 56 134.018505) (end 65.5 124.518505) (width 0.5) (layer B.Cu) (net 17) (status 10))
 (segment (start 56 135) (end 56 134.018505) (width 0.5) (layer B.Cu) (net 17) (status 30))
 (segment (start 65.5 115) (end 81.5 99) (width 0.5) (layer B.Cu) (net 17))
 (segment (start 65.5 124.518505) (end 65.5 115) (width 0.5) (layer B.Cu) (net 17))
 (segment (start 140 142.5) (end 146 142.5) (width 0.5) (layer B.Cu) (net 17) (status 20))
 (segment (start 121.5 124) (end 140 142.5) (width 0.5) (layer B.Cu) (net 17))
 (segment (start 116.709998 124) (end 121.5 124) (width 0.5) (layer B.Cu) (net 17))
 (segment (start 105.030001 112.320003) (end 116.709998 124) (width 0.5) (layer B.Cu) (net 17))
 (segment (start 105.030001 111.159999) (end 105.030001 112.320003) (width 0.5) (layer B.Cu) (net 17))
 (segment (start 95.38 110) (end 103.870002 110) (width 0.5) (layer B.Cu) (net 17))
 (segment (start 103.870002 110) (end 105.030001 111.159999) (width 0.5) (layer B.Cu) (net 17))
 (segment (start 93.62 111.76) (end 95.38 110) (width 0.5) (layer B.Cu) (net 17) (status 10))
 (segment (start 65.5 124.518505) (end 65.5 124.5) (width 0.5) (layer B.Cu) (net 17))
 (segment (start 55.018505 135) (end 54 136.018505) (width 0.5) (layer B.Cu) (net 17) (status 10))
 (segment (start 56 135) (end 55.018505 135) (width 0.5) (layer B.Cu) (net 17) (status 30))
 (segment (start 54 136.018505) (end 54 140.5) (width 0.5) (layer B.Cu) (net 17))
 (segment (start 54 140.5) (end 58 144.5) (width 0.5) (layer B.Cu) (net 17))
 (segment (start 73 144.5) (end 76 141.5) (width 0.5) (layer B.Cu) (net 17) (status 20))
 (segment (start 58 144.5) (end 73 144.5) (width 0.5) (layer B.Cu) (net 17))
 (segment (start 88.5 138.35) (end 88.5 137) (width 0.5) (layer B.Cu) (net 17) (status 20))
 (segment (start 85.35 141.5) (end 88.5 138.35) (width 0.5) (layer B.Cu) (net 17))
 (segment (start 76 141.5) (end 85.35 141.5) (width 0.5) (layer B.Cu) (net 17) (status 10))
 (segment (start 93.62 111.76) (end 89.88 115.5) (width 0.5) (layer B.Cu) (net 17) (status 10))
 (segment (start 89.88 115.5) (end 84 115.5) (width 0.5) (layer B.Cu) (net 17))
 (segment (start 81.5 113) (end 81.5 99) (width 0.5) (layer B.Cu) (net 17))
 (segment (start 84 115.5) (end 81.5 113) (width 0.5) (layer B.Cu) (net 17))
 (segment (start 81.5 85.5) (end 81.5 99) (width 0.5) (layer B.Cu) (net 17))
 (segment (start 90.5 76.5) (end 81.5 85.5) (width 0.5) (layer B.Cu) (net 17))
 (segment (start 90.5 66.5) (end 90.5 76.5) (width 0.5) (layer B.Cu) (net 17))
 (segment (start 98.5 58.5) (end 90.5 66.5) (width 0.5) (layer B.Cu) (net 17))
 (segment (start 106.5 59.15) (end 105.85 58.5) (width 0.5) (layer B.Cu) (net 17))
 (segment (start 105.85 58.5) (end 98.5 58.5) (width 0.5) (layer B.Cu) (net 17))
 (segment (start 106.5 60.5) (end 106.5 59.15) (width 0.5) (layer B.Cu) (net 17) (status 10))
 (segment (start 58.119999 136.349706) (end 58.650294 136.349706) (width 0.5) (layer B.Cu) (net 13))
 (segment (start 57.27 137.199705) (end 58.119999 136.349706) (width 0.5) (layer B.Cu) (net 13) (status 10))
 (segment (start 58.650294 136.349706) (end 75 120) (width 0.5) (layer B.Cu) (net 13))
 (segment (start 93 120) (end 101.24 111.76) (width 0.5) (layer B.Cu) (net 13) (status 20))
 (segment (start 75 120) (end 93 120) (width 0.5) (layer B.Cu) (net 13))
 (segment (start 58.54 139.399409) (end 75.439409 122.5) (width 0.5) (layer B.Cu) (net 11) (status 10))
 (segment (start 93.04 122.5) (end 103.78 111.76) (width 0.5) (layer B.Cu) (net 11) (status 20))
 (segment (start 75.439409 122.5) (end 93.04 122.5) (width 0.5) (layer B.Cu) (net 11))
 (segment (start 101.42 60.5) (end 101.42 94.42) (width 0.5) (layer B.Cu) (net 9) (status 10))
 (segment (start 106.32 99.32) (end 106.32 111.76) (width 0.5) (layer B.Cu) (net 9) (status 20))
 (segment (start 101.42 94.42) (end 106.32 99.32) (width 0.5) (layer B.Cu) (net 9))
 (segment (start 103.96 60.5) (end 103.96 93.46) (width 0.5) (layer B.Cu) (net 8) (status 10))
 (segment (start 108.86 98.36) (end 108.86 111.76) (width 0.5) (layer B.Cu) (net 8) (status 20))
 (segment (start 103.96 93.46) (end 108.86 98.36) (width 0.5) (layer B.Cu) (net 8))
 (segment (start 111.4 111.76) (end 134.14 134.5) (width 0.5) (layer B.Cu) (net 7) (status 10))
 (segment (start 141.469705 134.5) (end 147.27 140.300295) (width 0.5) (layer B.Cu) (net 7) (status 20))
 (segment (start 134.14 134.5) (end 141.469705 134.5) (width 0.5) (layer B.Cu) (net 7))
 (segment (start 148.54 138.100591) (end 142.939409 132.5) (width 0.5) (layer B.Cu) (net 5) (status 10))
 (segment (start 134.68 132.5) (end 113.94 111.76) (width 0.5) (layer B.Cu) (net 5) (status 20))
 (segment (start 142.939409 132.5) (end 134.68 132.5) (width 0.5) (layer B.Cu) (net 5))
 (segment (start 80.34 131.34) (end 80.5 131.5) (width 0.5) (layer B.Cu) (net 3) (status 30))
 (segment (start 76 131.34) (end 80.34 131.34) (width 0.5) (layer B.Cu) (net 3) (status 30))
 (segment (start 80.88 131.88) (end 80.5 131.5) (width 0.5) (layer B.Cu) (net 3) (status 30))
 (segment (start 80.88 137) (end 80.88 131.88) (width 0.5) (layer B.Cu) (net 3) (status 30))
 (segment (start 85 127) (end 86 127) (width 0.5) (layer B.Cu) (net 3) (status 20))
 (segment (start 80.5 131.5) (end 85 127) (width 0.5) (layer B.Cu) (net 3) (status 10))
 (segment (start 83.42 132.12) (end 85.54 130) (width 0.5) (layer B.Cu) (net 4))
 (segment (start 83.42 137) (end 83.42 132.12) (width 0.5) (layer B.Cu) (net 4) (status 10))
 (segment (start 85.54 130) (end 87 130) (width 0.5) (layer B.Cu) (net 4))
 (segment (start 88.54 128.46) (end 88.54 127) (width 0.5) (layer B.Cu) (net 4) (status 20))
 (segment (start 87 130) (end 88.54 128.46) (width 0.5) (layer B.Cu) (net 4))
 (segment (start 121.56 136.44) (end 121.5 136.5) (width 0.5) (layer B.Cu) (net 22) (status 30))
 (segment (start 121.56 127) (end 121.56 136.44) (width 0.5) (layer B.Cu) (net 22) (status 30))
 (segment (start 119.02 136.44) (end 118.96 136.5) (width 0.5) (layer B.Cu) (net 20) (status 30))
 (segment (start 119.02 127) (end 119.02 136.44) (width 0.5) (layer B.Cu) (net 20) (status 30))
 (segment (start 116.48 136.44) (end 116.42 136.5) (width 0.5) (layer B.Cu) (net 19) (status 30))
 (segment (start 116.48 127) (end 116.48 136.44) (width 0.5) (layer B.Cu) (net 19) (status 30))
 (segment (start 113.94 136.44) (end 113.88 136.5) (width 0.5) (layer B.Cu) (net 18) (status 30))
 (segment (start 113.94 127) (end 113.94 136.44) (width 0.5) (layer B.Cu) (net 18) (status 30))
 (segment (start 111.4 136.44) (end 111.34 136.5) (width 0.5) (layer B.Cu) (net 16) (status 30))
 (segment (start 111.4 127) (end 111.4 136.44) (width 0.5) (layer B.Cu) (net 16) (status 30))
 (segment (start 108.86 136.44) (end 108.8 136.5) (width 0.5) (layer B.Cu) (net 15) (status 30))
 (segment (start 108.86 127) (end 108.86 136.44) (width 0.5) (layer B.Cu) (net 15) (status 30))
 (segment (start 106.32 136.44) (end 106.26 136.5) (width 0.5) (layer B.Cu) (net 14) (status 30))
 (segment (start 106.32 127) (end 106.32 136.44) (width 0.5) (layer B.Cu) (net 14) (status 30))
 (segment (start 103.78 136.44) (end 103.72 136.5) (width 0.5) (layer B.Cu) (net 12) (status 30))
 (segment (start 103.78 127) (end 103.78 136.44) (width 0.5) (layer B.Cu) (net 12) (status 30))
 (segment (start 101.24 136.44) (end 101.18 136.5) (width 0.5) (layer B.Cu) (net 10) (status 30))
 (segment (start 101.24 127) (end 101.24 136.44) (width 0.5) (layer B.Cu) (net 10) (status 30))
 (segment (start 99.568 72.568) (end 99.568 101.032) (width 0.5) (layer B.Cu) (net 1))
 (segment (start 96.5 69.5) (end 99.568 72.568) (width 0.5) (layer B.Cu) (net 1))
 (segment (start 94.5 69.5) (end 96.5 69.5) (width 0.5) (layer B.Cu) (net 1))
 (segment (start 97.1 103.5) (end 95 103.5) (width 0.5) (layer B.Cu) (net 1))
 (segment (start 99.568 101.032) (end 97.1 103.5) (width 0.5) (layer B.Cu) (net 1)))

